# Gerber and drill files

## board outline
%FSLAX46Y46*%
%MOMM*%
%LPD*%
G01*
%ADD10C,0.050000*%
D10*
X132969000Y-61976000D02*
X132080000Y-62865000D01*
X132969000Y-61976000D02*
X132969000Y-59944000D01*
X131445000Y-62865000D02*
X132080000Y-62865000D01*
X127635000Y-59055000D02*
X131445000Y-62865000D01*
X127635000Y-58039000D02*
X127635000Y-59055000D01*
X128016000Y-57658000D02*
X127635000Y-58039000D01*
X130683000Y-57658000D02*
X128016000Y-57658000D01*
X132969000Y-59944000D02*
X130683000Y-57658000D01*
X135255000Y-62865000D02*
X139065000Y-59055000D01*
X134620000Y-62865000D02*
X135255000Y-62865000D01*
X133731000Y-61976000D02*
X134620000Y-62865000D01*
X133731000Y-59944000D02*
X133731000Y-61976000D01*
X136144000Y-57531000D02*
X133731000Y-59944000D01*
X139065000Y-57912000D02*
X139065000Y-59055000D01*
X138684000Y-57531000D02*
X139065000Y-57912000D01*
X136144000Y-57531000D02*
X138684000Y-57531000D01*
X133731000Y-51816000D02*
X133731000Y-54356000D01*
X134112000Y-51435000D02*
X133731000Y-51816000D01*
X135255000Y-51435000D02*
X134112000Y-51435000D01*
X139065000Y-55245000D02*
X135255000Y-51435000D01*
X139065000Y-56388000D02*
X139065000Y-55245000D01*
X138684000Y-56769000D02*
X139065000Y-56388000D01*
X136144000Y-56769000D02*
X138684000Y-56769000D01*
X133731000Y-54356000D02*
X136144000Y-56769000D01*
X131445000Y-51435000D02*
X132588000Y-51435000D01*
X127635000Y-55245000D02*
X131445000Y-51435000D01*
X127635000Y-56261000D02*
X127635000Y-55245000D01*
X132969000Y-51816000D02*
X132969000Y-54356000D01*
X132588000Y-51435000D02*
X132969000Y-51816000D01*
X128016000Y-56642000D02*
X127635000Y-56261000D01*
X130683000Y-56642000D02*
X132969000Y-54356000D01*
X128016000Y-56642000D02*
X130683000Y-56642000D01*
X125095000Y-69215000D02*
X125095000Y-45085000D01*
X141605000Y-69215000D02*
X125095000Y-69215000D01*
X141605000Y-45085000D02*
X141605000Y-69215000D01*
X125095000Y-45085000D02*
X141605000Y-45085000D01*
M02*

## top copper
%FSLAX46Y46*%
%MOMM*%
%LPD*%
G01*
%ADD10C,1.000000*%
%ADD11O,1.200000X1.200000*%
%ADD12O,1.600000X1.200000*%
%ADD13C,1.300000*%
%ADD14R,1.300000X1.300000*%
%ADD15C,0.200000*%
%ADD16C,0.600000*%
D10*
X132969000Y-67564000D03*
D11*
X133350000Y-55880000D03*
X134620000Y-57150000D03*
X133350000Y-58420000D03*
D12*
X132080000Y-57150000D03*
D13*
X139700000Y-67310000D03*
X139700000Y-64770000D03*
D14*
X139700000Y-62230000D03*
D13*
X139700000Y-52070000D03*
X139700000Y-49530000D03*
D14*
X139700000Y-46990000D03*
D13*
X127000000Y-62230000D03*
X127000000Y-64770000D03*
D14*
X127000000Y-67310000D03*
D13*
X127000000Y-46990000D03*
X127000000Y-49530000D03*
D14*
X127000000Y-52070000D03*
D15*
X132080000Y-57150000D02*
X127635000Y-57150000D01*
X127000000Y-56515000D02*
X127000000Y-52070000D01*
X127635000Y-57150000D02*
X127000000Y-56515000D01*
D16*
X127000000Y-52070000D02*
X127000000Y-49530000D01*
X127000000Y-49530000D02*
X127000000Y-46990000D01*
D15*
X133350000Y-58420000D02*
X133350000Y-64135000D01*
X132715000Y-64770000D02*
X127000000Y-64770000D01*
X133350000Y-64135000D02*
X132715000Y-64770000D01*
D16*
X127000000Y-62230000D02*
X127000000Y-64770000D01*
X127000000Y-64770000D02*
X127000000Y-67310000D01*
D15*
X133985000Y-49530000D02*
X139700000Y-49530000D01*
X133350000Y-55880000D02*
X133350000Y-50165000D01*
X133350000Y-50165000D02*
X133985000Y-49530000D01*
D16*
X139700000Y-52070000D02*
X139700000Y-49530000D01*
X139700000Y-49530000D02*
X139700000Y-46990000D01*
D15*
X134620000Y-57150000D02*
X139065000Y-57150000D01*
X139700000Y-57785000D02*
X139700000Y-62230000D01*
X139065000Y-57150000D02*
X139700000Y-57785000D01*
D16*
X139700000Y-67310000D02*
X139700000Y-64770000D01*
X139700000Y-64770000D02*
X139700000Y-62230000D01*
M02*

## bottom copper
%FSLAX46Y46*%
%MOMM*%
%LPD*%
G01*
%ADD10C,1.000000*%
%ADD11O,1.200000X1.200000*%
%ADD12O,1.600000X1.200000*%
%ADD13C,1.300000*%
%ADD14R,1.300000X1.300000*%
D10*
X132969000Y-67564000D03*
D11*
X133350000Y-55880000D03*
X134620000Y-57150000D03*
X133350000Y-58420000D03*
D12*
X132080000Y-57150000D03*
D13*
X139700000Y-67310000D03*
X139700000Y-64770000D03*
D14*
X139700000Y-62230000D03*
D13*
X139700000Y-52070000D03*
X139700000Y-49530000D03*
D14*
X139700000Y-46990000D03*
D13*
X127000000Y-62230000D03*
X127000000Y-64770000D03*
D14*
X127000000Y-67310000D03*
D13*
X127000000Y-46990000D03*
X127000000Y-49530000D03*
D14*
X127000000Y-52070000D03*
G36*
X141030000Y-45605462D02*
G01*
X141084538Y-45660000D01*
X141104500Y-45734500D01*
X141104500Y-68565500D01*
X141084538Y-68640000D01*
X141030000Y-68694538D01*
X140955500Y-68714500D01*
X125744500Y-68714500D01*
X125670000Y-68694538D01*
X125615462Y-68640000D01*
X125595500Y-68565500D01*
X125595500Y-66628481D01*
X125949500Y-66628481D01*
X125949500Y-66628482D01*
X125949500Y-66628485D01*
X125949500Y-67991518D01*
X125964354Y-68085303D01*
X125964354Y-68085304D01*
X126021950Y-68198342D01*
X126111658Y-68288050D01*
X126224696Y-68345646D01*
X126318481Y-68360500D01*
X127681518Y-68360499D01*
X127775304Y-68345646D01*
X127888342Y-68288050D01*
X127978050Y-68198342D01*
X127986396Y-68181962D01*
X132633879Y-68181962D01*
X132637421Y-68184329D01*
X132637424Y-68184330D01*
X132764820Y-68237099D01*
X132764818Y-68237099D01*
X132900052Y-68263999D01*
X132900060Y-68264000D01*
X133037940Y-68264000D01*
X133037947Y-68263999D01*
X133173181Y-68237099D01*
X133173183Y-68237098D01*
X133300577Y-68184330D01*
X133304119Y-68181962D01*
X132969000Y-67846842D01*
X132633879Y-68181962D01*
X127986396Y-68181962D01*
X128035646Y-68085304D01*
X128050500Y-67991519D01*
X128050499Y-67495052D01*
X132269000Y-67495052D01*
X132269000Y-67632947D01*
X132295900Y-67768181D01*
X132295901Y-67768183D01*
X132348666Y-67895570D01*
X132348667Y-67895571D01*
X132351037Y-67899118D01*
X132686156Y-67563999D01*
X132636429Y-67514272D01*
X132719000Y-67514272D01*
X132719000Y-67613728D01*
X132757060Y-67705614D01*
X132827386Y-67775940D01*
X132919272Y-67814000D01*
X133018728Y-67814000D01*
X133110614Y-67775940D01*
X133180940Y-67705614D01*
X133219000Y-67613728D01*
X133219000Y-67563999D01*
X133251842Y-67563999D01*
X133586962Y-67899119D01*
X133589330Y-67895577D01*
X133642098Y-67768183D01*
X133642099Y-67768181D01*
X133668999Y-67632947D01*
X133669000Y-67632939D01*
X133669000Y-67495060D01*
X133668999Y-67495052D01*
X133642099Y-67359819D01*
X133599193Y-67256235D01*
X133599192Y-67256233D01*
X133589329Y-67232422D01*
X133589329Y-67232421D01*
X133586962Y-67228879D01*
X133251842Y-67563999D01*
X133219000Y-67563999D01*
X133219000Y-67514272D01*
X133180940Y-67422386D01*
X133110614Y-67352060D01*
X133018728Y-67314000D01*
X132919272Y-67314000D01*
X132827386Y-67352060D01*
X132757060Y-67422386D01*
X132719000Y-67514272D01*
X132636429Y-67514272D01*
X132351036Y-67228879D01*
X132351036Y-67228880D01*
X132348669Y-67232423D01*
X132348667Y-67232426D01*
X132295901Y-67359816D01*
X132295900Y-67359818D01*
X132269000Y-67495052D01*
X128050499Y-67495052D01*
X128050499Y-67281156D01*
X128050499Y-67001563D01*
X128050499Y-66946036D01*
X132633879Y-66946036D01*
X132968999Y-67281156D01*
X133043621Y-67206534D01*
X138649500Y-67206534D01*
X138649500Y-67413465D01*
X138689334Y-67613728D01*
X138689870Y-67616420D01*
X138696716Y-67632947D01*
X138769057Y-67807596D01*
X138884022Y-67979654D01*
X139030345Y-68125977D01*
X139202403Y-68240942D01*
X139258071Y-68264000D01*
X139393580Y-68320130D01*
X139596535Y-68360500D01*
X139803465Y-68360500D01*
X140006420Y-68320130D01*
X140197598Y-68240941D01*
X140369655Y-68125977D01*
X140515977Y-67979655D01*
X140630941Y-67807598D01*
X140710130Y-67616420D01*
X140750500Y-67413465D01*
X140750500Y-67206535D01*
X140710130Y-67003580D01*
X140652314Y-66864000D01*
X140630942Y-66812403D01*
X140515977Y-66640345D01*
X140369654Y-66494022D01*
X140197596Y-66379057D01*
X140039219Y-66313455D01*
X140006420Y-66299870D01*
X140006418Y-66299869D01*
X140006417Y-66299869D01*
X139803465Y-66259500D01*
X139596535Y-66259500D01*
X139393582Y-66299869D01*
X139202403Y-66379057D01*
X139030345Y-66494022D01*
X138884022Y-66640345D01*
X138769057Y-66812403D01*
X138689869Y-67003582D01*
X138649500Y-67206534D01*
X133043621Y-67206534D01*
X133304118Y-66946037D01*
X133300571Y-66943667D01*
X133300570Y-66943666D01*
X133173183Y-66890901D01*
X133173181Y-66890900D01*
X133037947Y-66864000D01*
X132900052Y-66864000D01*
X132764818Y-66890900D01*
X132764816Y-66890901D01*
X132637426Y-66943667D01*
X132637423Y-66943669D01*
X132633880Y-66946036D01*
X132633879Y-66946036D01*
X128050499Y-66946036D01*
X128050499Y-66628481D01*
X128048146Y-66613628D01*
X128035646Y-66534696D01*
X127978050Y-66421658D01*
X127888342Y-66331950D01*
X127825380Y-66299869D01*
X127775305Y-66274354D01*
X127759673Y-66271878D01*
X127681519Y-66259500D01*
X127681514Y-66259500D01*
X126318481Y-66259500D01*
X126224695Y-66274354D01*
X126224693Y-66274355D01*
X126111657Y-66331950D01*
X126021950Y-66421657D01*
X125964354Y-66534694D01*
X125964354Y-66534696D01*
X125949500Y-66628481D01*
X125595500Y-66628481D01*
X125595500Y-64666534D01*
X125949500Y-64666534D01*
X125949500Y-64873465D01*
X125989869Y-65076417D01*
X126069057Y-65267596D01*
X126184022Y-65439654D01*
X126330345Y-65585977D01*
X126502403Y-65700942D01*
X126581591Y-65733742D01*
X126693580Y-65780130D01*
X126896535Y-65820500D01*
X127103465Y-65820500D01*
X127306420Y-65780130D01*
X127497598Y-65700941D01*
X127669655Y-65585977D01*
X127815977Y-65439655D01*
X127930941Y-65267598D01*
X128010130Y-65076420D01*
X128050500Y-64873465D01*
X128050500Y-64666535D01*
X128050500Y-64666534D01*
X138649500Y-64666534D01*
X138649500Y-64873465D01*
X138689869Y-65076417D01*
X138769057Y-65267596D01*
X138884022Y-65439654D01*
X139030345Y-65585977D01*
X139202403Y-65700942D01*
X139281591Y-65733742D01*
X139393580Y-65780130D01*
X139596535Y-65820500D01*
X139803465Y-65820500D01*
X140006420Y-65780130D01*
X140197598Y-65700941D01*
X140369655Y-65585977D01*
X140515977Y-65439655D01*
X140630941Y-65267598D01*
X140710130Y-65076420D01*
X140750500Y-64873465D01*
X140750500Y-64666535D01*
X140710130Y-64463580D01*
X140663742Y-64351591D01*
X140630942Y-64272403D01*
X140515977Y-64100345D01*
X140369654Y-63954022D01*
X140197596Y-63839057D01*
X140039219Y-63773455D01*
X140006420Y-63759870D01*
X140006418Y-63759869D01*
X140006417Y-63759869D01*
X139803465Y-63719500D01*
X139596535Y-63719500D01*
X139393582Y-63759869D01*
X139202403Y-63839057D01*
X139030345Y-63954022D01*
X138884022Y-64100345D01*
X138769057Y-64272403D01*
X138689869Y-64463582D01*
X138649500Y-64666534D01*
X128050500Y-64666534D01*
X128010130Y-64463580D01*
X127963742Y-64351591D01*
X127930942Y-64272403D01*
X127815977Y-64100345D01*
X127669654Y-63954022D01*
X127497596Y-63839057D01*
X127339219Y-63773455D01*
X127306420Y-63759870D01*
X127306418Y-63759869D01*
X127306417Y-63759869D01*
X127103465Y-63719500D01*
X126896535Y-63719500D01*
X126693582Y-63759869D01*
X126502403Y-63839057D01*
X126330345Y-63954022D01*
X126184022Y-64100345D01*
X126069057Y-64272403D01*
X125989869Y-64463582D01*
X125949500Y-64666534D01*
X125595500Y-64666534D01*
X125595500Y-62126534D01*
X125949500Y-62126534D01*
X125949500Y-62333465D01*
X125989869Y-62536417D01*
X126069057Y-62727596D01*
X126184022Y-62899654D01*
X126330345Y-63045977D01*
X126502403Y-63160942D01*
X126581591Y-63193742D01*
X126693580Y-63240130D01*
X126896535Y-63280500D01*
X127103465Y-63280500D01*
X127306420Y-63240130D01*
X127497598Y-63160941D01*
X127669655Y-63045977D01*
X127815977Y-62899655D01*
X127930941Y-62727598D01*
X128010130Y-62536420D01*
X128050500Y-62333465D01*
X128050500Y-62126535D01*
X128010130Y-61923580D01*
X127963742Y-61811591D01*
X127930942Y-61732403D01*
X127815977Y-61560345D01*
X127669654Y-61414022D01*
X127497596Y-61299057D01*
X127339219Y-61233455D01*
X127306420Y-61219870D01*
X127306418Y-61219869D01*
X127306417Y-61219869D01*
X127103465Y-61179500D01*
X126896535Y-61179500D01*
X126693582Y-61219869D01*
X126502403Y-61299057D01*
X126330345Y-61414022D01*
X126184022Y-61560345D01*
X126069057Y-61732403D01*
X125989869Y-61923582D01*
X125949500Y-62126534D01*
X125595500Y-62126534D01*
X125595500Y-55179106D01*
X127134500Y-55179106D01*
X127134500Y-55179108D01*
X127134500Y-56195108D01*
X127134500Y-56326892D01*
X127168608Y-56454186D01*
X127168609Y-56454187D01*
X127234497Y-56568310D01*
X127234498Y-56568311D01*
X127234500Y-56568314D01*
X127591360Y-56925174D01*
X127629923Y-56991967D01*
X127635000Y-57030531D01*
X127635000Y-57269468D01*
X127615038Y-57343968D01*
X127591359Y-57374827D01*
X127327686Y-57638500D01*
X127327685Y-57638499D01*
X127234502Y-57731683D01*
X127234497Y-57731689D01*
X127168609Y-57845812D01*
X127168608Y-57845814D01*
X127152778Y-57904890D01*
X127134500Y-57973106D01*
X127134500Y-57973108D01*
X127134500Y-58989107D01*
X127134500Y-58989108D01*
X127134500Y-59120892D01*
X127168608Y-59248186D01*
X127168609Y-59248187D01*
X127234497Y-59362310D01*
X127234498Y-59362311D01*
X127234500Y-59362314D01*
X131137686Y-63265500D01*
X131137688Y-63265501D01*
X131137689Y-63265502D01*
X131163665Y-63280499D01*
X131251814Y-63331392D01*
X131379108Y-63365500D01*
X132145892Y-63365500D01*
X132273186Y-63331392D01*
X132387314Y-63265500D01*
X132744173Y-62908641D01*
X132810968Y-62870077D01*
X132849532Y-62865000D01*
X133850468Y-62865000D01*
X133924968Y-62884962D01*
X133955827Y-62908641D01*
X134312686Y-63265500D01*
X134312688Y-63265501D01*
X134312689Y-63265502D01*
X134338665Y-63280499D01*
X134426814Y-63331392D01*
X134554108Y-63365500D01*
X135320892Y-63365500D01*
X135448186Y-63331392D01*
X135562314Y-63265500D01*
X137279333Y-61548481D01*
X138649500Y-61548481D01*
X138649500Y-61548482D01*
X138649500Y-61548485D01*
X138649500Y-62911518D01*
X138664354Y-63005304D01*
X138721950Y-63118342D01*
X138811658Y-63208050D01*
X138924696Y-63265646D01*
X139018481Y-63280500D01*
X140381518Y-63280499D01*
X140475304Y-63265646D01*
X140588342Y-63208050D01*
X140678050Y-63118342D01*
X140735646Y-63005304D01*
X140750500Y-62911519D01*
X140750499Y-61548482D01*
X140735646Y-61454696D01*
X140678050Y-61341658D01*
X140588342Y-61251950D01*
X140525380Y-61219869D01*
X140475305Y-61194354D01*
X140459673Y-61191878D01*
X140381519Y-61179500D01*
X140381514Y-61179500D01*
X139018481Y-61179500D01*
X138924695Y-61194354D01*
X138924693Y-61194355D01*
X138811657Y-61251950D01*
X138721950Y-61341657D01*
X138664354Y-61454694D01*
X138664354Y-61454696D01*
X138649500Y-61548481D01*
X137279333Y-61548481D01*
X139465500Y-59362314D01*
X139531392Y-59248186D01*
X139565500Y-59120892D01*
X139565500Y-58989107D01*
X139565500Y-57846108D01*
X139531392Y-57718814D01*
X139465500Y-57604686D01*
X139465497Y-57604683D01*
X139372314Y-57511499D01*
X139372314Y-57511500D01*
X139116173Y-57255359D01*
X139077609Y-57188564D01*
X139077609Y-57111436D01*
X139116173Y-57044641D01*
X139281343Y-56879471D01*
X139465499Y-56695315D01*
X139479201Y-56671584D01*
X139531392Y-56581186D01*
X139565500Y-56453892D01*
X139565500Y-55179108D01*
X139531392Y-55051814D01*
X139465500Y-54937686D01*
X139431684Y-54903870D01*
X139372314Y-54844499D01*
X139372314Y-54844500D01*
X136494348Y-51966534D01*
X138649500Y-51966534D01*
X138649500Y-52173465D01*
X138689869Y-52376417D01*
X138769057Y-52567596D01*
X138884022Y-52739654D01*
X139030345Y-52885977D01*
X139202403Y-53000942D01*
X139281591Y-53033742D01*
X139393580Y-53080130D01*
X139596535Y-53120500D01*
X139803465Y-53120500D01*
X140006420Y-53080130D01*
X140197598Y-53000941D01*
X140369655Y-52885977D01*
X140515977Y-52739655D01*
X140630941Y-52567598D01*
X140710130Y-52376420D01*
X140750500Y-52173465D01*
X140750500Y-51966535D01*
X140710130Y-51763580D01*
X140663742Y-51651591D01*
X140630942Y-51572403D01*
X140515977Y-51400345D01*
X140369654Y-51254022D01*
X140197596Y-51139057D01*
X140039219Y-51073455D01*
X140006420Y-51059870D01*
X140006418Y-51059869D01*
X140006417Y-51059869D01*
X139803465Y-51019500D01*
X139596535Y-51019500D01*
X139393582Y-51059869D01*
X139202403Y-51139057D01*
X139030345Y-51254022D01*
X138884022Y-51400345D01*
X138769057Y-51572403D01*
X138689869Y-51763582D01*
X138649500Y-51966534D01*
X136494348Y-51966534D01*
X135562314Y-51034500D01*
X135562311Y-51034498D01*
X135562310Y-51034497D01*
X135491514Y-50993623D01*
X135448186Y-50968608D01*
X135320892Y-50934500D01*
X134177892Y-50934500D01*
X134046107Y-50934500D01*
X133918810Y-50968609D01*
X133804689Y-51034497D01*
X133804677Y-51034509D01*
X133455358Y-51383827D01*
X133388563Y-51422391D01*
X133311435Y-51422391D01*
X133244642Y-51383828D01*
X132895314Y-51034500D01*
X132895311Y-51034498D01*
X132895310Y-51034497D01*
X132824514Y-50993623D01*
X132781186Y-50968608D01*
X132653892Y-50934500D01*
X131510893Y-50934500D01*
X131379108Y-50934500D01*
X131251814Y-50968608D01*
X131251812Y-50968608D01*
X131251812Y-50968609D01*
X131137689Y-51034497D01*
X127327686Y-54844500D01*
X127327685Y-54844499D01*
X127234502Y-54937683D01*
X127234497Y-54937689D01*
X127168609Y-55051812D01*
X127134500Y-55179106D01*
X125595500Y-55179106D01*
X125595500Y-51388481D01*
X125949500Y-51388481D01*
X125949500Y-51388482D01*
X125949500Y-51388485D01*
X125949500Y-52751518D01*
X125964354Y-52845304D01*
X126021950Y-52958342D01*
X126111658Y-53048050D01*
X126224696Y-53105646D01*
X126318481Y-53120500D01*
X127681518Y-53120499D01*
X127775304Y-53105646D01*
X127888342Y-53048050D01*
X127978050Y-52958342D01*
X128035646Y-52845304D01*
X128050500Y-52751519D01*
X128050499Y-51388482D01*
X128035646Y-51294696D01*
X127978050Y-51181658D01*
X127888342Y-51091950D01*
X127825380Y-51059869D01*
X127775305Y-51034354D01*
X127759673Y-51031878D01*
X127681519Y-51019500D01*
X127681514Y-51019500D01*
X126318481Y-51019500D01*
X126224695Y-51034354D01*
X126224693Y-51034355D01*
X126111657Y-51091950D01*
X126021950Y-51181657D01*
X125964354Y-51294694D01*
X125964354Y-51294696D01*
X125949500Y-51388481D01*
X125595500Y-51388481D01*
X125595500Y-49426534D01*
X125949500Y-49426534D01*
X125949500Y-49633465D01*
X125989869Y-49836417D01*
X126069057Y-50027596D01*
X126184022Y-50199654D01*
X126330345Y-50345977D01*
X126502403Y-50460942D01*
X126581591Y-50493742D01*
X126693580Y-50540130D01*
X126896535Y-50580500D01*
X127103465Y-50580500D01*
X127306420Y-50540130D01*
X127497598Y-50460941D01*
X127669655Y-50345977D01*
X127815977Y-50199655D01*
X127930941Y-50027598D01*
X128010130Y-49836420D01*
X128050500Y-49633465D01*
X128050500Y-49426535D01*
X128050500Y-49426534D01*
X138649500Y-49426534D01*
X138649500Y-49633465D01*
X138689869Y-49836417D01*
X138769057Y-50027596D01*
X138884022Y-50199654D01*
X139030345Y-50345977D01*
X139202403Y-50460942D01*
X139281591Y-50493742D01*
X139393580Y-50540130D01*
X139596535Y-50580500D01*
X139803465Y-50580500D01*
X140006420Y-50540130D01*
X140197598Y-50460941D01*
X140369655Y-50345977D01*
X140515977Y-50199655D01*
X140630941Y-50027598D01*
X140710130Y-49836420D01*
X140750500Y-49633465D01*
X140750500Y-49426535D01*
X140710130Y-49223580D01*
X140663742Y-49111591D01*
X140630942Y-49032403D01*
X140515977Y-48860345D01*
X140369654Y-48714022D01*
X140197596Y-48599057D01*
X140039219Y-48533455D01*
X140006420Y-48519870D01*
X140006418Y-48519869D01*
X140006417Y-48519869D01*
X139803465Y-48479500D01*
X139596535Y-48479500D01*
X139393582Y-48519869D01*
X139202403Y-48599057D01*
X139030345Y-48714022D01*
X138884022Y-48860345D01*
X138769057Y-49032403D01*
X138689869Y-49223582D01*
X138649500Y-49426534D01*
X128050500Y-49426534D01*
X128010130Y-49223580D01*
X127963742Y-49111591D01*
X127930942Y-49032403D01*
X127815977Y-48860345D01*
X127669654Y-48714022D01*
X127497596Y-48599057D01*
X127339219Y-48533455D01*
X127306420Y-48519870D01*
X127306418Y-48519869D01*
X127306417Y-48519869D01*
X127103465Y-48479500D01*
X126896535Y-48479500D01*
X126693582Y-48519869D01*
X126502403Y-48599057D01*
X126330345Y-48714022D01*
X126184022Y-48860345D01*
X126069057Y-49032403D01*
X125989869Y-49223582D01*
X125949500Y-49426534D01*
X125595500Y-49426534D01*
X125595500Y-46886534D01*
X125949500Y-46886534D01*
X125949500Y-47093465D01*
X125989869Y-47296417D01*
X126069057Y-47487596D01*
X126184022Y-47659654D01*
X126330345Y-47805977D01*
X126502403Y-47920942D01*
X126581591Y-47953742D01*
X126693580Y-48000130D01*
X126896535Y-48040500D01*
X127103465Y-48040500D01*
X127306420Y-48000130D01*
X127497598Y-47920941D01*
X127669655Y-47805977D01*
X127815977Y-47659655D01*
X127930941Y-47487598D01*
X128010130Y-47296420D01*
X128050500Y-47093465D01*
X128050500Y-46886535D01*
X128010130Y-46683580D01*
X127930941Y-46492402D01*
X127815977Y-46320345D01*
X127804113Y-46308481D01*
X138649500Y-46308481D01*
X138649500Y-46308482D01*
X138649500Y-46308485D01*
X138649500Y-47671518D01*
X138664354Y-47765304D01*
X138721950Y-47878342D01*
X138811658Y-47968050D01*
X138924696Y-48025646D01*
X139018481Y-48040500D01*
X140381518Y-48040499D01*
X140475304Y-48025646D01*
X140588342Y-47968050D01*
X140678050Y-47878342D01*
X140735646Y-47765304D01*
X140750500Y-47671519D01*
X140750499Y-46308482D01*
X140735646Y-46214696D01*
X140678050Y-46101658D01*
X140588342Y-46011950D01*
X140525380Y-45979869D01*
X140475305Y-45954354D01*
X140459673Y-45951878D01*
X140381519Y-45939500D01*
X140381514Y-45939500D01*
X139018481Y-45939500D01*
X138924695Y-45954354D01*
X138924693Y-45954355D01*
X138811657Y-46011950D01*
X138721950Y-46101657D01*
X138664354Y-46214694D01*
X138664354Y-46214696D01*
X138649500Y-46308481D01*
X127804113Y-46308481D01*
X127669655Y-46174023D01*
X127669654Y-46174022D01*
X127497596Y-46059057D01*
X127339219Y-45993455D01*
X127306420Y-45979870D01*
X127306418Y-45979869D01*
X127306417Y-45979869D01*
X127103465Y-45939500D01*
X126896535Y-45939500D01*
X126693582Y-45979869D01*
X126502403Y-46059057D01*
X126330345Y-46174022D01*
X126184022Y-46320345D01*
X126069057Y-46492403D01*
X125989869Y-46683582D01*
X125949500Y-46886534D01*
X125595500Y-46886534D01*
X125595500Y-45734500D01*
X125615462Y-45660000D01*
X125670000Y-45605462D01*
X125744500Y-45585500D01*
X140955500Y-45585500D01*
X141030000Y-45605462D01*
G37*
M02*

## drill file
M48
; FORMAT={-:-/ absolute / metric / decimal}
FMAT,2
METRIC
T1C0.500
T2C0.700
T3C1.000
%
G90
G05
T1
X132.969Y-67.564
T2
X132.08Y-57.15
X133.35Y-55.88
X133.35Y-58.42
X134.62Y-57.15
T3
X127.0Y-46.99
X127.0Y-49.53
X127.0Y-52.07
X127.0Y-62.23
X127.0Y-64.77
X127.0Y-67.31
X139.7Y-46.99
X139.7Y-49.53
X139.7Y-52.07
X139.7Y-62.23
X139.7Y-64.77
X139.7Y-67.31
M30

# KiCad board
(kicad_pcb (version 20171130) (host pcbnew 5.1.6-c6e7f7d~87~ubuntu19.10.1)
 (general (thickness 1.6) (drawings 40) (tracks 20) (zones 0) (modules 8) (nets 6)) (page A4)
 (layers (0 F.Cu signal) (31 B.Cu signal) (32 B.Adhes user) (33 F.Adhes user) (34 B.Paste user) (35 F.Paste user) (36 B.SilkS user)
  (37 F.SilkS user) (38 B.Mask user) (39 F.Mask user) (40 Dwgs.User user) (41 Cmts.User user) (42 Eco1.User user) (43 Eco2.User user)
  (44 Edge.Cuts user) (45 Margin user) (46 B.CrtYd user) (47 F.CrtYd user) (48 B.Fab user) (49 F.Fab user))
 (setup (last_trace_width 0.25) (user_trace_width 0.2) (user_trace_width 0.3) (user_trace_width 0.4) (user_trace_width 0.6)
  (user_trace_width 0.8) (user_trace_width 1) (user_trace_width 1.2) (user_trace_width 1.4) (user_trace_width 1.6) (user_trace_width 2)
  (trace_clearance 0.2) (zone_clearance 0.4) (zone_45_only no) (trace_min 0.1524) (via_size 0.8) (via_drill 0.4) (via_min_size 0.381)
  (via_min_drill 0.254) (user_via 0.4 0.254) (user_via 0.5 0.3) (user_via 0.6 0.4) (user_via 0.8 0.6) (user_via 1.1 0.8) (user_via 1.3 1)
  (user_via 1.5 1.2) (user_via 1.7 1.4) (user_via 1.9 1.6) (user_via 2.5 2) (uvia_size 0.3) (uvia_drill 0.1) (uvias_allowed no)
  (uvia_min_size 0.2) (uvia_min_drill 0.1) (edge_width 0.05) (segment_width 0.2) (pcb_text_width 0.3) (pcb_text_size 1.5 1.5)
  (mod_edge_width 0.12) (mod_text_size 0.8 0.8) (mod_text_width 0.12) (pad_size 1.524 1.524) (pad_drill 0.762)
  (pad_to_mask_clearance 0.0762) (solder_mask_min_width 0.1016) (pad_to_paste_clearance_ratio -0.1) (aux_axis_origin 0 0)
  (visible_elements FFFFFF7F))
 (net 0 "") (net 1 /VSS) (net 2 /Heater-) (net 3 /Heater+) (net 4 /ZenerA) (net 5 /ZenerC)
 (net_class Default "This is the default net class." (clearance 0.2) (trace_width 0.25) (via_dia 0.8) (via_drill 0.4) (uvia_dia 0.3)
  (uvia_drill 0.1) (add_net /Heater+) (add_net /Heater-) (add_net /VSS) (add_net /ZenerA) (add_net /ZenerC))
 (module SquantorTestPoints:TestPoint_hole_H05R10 (layer F.Cu) (at 132.969 67.564)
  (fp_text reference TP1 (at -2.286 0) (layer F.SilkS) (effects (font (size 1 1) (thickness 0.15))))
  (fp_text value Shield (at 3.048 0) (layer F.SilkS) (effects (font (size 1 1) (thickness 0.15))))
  (pad 1 thru_hole circle (at 0 0) (size 1 1) (drill 0.5) (layers *.Cu *.Mask) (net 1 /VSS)))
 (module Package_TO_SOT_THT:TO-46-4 (layer F.Cu) (at 132.08 57.15)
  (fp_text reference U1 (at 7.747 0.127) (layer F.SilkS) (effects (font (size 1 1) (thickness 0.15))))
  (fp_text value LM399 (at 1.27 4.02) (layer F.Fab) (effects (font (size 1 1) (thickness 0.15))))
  (pad 4 thru_hole oval (at 1.27 -1.27) (size 1.2 1.2) (drill 0.7) (layers *.Cu *.Mask) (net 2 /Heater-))
  (pad 3 thru_hole oval (at 2.54 0) (size 1.2 1.2) (drill 0.7) (layers *.Cu *.Mask) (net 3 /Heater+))
  (pad 2 thru_hole oval (at 1.27 1.27) (size 1.2 1.2) (drill 0.7) (layers *.Cu *.Mask) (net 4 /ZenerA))
  (pad 1 thru_hole oval (at 0 0) (size 1.6 1.2) (drill 0.7) (layers *.Cu *.Mask) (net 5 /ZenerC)))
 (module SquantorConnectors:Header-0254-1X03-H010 (layer F.Cu) (at 139.7 64.77 270)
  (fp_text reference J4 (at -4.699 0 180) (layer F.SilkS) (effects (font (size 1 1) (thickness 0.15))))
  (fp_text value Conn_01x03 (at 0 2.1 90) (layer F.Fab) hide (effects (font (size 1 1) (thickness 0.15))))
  (pad 3 thru_hole circle (at 2.54 0 90) (size 1.3 1.3) (drill 1) (layers *.Cu *.Mask) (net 3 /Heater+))
  (pad 2 thru_hole circle (at 0 0 90) (size 1.3 1.3) (drill 1) (layers *.Cu *.Mask) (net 3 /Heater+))
  (pad 1 thru_hole rect (at -2.54 0 90) (size 1.3 1.3) (drill 1) (layers *.Cu *.Mask) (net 3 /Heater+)))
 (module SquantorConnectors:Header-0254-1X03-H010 (layer F.Cu) (at 139.7 49.53 270)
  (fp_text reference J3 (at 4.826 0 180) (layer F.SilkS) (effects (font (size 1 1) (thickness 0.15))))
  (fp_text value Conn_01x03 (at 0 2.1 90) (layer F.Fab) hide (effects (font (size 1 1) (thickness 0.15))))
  (pad 3 thru_hole circle (at 2.54 0 90) (size 1.3 1.3) (drill 1) (layers *.Cu *.Mask) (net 2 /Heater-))
  (pad 2 thru_hole circle (at 0 0 90) (size 1.3 1.3) (drill 1) (layers *.Cu *.Mask) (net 2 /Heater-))
  (pad 1 thru_hole rect (at -2.54 0 90) (size 1.3 1.3) (drill 1) (layers *.Cu *.Mask) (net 2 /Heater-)))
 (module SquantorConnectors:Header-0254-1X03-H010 (layer F.Cu) (at 127 64.77 90)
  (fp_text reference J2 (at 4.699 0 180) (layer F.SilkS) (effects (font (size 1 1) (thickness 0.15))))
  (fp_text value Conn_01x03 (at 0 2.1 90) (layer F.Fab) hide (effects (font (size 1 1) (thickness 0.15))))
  (pad 3 thru_hole circle (at 2.54 0 270) (size 1.3 1.3) (drill 1) (layers *.Cu *.Mask) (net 4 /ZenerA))
  (pad 2 thru_hole circle (at 0 0 270) (size 1.3 1.3) (drill 1) (layers *.Cu *.Mask) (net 4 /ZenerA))
  (pad 1 thru_hole rect (at -2.54 0 270) (size 1.3 1.3) (drill 1) (layers *.Cu *.Mask) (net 4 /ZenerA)))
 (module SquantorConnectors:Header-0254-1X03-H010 (layer F.Cu) (at 127 49.53 90)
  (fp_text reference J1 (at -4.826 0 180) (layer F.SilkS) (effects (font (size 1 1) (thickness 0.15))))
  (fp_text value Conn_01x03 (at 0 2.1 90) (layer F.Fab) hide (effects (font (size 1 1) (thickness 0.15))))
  (pad 3 thru_hole circle (at 2.54 0 270) (size 1.3 1.3) (drill 1) (layers *.Cu *.Mask) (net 5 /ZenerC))
  (pad 2 thru_hole circle (at 0 0 270) (size 1.3 1.3) (drill 1) (layers *.Cu *.Mask) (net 5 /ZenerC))
  (pad 1 thru_hole rect (at -2.54 0 270) (size 1.3 1.3) (drill 1) (layers *.Cu *.Mask) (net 5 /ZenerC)))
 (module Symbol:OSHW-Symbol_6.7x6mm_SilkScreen (layer B.Cu) (at 133.35 48.387 180)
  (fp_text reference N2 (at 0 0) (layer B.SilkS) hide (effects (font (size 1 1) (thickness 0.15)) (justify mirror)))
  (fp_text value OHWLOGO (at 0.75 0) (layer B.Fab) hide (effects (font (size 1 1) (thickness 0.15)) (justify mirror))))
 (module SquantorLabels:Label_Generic (layer B.Cu) (at 133.858 64.77 180)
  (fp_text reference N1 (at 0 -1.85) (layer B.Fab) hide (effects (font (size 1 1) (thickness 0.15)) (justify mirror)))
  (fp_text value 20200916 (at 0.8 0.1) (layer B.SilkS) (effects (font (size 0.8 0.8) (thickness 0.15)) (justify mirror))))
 (gr_line (start 132.969 61.976) (end 132.08 62.865) (layer Edge.Cuts) (width 0.05))
 (gr_line (start 132.969 61.976) (end 132.969 59.944) (layer Edge.Cuts) (width 0.05))
 (gr_line (start 131.445 62.865) (end 132.08 62.865) (layer Edge.Cuts) (width 0.05))
 (gr_line (start 127.635 59.055) (end 131.445 62.865) (layer Edge.Cuts) (width 0.05))
 (gr_line (start 127.635 58.039) (end 127.635 59.055) (layer Edge.Cuts) (width 0.05))
 (gr_line (start 128.016 57.658) (end 127.635 58.039) (layer Edge.Cuts) (width 0.05))
 (gr_line (start 130.683 57.658) (end 128.016 57.658) (layer Edge.Cuts) (width 0.05))
 (gr_line (start 132.969 59.944) (end 130.683 57.658) (layer Edge.Cuts) (width 0.05))
 (gr_line (start 135.255 62.865) (end 139.065 59.055) (layer Edge.Cuts) (width 0.05))
 (gr_line (start 134.62 62.865) (end 135.255 62.865) (layer Edge.Cuts) (width 0.05))
 (gr_line (start 133.731 61.976) (end 134.62 62.865) (layer Edge.Cuts) (width 0.05))
 (gr_line (start 133.731 59.944) (end 133.731 61.976) (layer Edge.Cuts) (width 0.05))
 (gr_line (start 136.144 57.531) (end 133.731 59.944) (layer Edge.Cuts) (width 0.05))
 (gr_line (start 139.065 57.912) (end 139.065 59.055) (layer Edge.Cuts) (width 0.05))
 (gr_line (start 138.684 57.531) (end 139.065 57.912) (layer Edge.Cuts) (width 0.05))
 (gr_line (start 136.144 57.531) (end 138.684 57.531) (layer Edge.Cuts) (width 0.05))
 (gr_line (start 133.731 51.816) (end 133.731 54.356) (layer Edge.Cuts) (width 0.05))
 (gr_line (start 134.112 51.435) (end 133.731 51.816) (layer Edge.Cuts) (width 0.05))
 (gr_line (start 135.255 51.435) (end 134.112 51.435) (layer Edge.Cuts) (width 0.05))
 (gr_line (start 139.065 55.245) (end 135.255 51.435) (layer Edge.Cuts) (width 0.05))
 (gr_line (start 139.065 56.388) (end 139.065 55.245) (layer Edge.Cuts) (width 0.05))
 (gr_line (start 138.684 56.769) (end 139.065 56.388) (layer Edge.Cuts) (width 0.05))
 (gr_line (start 136.144 56.769) (end 138.684 56.769) (layer Edge.Cuts) (width 0.05))
 (gr_line (start 133.731 54.356) (end 136.144 56.769) (layer Edge.Cuts) (width 0.05))
 (gr_line (start 131.445 51.435) (end 132.588 51.435) (layer Edge.Cuts) (width 0.05))
 (gr_line (start 127.635 55.245) (end 131.445 51.435) (layer Edge.Cuts) (width 0.05))
 (gr_line (start 127.635 56.261) (end 127.635 55.245) (layer Edge.Cuts) (width 0.05))
 (gr_line (start 132.969 51.816) (end 132.969 54.356) (layer Edge.Cuts) (width 0.05))
 (gr_line (start 132.588 51.435) (end 132.969 51.816) (layer Edge.Cuts) (width 0.05))
 (gr_line (start 128.016 56.642) (end 127.635 56.261) (layer Edge.Cuts) (width 0.05))
 (gr_line (start 130.683 56.642) (end 132.969 54.356) (layer Edge.Cuts) (width 0.05))
 (gr_line (start 128.016 56.642) (end 130.683 56.642) (layer Edge.Cuts) (width 0.05))
 (gr_line (start 125.095 69.215) (end 125.095 45.085) (layer Edge.Cuts) (width 0.05))
 (gr_line (start 141.605 69.215) (end 125.095 69.215) (layer Edge.Cuts) (width 0.05))
 (gr_line (start 141.605 45.085) (end 141.605 69.215) (layer Edge.Cuts) (width 0.05))
 (gr_line (start 125.095 45.085) (end 141.605 45.085) (layer Edge.Cuts) (width 0.05))
 (segment (start 132.08 57.15) (end 127.635 57.15) (width 0.2) (layer F.Cu) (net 5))
 (segment (start 127 56.515) (end 127 52.07) (width 0.2) (layer F.Cu) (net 5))
 (segment (start 127.635 57.15) (end 127 56.515) (width 0.2) (layer F.Cu) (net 5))
 (segment (start 127 52.07) (end 127 49.53) (width 0.6) (layer F.Cu) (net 5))
 (segment (start 127 49.53) (end 127 46.99) (width 0.6) (layer F.Cu) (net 5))
 (segment (start 133.35 58.42) (end 133.35 64.135) (width 0.2) (layer F.Cu) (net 4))
 (segment (start 132.715 64.77) (end 127 64.77) (width 0.2) (layer F.Cu) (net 4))
 (segment (start 133.35 64.135) (end 132.715 64.77) (width 0.2) (layer F.Cu) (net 4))
 (segment (start 127 62.23) (end 127 64.77) (width 0.6) (layer F.Cu) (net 4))
 (segment (start 127 64.77) (end 127 67.31) (width 0.6) (layer F.Cu) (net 4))
 (segment (start 133.985 49.53) (end 139.7 49.53) (width 0.2) (layer F.Cu) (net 2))
 (segment (start 133.35 55.88) (end 133.35 50.165) (width 0.2) (layer F.Cu) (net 2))
 (segment (start 133.35 50.165) (end 133.985 49.53) (width 0.2) (layer F.Cu) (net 2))
 (segment (start 139.7 52.07) (end 139.7 49.53) (width 0.6) (layer F.Cu) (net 2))
 (segment (start 139.7 49.53) (end 139.7 46.99) (width 0.6) (layer F.Cu) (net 2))
 (segment (start 134.62 57.15) (end 139.065 57.15) (width 0.2) (layer F.Cu) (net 3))
 (segment (start 139.7 57.785) (end 139.7 62.23) (width 0.2) (layer F.Cu) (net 3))
 (segment (start 139.065 57.15) (end 139.7 57.785) (width 0.2) (layer F.Cu) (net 3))
 (segment (start 139.7 67.31) (end 139.7 64.77) (width 0.6) (layer F.Cu) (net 3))
 (segment (start 139.7 64.77) (end 139.7 62.23) (width 0.6) (layer F.Cu) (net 3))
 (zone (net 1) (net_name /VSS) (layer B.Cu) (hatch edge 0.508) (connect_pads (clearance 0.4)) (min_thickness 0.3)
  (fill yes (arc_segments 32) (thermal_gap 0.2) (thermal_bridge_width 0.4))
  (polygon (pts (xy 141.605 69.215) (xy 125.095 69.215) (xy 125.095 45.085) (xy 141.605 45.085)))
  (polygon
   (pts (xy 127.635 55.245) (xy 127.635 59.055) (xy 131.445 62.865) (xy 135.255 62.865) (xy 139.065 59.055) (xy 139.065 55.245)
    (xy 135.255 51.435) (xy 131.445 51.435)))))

